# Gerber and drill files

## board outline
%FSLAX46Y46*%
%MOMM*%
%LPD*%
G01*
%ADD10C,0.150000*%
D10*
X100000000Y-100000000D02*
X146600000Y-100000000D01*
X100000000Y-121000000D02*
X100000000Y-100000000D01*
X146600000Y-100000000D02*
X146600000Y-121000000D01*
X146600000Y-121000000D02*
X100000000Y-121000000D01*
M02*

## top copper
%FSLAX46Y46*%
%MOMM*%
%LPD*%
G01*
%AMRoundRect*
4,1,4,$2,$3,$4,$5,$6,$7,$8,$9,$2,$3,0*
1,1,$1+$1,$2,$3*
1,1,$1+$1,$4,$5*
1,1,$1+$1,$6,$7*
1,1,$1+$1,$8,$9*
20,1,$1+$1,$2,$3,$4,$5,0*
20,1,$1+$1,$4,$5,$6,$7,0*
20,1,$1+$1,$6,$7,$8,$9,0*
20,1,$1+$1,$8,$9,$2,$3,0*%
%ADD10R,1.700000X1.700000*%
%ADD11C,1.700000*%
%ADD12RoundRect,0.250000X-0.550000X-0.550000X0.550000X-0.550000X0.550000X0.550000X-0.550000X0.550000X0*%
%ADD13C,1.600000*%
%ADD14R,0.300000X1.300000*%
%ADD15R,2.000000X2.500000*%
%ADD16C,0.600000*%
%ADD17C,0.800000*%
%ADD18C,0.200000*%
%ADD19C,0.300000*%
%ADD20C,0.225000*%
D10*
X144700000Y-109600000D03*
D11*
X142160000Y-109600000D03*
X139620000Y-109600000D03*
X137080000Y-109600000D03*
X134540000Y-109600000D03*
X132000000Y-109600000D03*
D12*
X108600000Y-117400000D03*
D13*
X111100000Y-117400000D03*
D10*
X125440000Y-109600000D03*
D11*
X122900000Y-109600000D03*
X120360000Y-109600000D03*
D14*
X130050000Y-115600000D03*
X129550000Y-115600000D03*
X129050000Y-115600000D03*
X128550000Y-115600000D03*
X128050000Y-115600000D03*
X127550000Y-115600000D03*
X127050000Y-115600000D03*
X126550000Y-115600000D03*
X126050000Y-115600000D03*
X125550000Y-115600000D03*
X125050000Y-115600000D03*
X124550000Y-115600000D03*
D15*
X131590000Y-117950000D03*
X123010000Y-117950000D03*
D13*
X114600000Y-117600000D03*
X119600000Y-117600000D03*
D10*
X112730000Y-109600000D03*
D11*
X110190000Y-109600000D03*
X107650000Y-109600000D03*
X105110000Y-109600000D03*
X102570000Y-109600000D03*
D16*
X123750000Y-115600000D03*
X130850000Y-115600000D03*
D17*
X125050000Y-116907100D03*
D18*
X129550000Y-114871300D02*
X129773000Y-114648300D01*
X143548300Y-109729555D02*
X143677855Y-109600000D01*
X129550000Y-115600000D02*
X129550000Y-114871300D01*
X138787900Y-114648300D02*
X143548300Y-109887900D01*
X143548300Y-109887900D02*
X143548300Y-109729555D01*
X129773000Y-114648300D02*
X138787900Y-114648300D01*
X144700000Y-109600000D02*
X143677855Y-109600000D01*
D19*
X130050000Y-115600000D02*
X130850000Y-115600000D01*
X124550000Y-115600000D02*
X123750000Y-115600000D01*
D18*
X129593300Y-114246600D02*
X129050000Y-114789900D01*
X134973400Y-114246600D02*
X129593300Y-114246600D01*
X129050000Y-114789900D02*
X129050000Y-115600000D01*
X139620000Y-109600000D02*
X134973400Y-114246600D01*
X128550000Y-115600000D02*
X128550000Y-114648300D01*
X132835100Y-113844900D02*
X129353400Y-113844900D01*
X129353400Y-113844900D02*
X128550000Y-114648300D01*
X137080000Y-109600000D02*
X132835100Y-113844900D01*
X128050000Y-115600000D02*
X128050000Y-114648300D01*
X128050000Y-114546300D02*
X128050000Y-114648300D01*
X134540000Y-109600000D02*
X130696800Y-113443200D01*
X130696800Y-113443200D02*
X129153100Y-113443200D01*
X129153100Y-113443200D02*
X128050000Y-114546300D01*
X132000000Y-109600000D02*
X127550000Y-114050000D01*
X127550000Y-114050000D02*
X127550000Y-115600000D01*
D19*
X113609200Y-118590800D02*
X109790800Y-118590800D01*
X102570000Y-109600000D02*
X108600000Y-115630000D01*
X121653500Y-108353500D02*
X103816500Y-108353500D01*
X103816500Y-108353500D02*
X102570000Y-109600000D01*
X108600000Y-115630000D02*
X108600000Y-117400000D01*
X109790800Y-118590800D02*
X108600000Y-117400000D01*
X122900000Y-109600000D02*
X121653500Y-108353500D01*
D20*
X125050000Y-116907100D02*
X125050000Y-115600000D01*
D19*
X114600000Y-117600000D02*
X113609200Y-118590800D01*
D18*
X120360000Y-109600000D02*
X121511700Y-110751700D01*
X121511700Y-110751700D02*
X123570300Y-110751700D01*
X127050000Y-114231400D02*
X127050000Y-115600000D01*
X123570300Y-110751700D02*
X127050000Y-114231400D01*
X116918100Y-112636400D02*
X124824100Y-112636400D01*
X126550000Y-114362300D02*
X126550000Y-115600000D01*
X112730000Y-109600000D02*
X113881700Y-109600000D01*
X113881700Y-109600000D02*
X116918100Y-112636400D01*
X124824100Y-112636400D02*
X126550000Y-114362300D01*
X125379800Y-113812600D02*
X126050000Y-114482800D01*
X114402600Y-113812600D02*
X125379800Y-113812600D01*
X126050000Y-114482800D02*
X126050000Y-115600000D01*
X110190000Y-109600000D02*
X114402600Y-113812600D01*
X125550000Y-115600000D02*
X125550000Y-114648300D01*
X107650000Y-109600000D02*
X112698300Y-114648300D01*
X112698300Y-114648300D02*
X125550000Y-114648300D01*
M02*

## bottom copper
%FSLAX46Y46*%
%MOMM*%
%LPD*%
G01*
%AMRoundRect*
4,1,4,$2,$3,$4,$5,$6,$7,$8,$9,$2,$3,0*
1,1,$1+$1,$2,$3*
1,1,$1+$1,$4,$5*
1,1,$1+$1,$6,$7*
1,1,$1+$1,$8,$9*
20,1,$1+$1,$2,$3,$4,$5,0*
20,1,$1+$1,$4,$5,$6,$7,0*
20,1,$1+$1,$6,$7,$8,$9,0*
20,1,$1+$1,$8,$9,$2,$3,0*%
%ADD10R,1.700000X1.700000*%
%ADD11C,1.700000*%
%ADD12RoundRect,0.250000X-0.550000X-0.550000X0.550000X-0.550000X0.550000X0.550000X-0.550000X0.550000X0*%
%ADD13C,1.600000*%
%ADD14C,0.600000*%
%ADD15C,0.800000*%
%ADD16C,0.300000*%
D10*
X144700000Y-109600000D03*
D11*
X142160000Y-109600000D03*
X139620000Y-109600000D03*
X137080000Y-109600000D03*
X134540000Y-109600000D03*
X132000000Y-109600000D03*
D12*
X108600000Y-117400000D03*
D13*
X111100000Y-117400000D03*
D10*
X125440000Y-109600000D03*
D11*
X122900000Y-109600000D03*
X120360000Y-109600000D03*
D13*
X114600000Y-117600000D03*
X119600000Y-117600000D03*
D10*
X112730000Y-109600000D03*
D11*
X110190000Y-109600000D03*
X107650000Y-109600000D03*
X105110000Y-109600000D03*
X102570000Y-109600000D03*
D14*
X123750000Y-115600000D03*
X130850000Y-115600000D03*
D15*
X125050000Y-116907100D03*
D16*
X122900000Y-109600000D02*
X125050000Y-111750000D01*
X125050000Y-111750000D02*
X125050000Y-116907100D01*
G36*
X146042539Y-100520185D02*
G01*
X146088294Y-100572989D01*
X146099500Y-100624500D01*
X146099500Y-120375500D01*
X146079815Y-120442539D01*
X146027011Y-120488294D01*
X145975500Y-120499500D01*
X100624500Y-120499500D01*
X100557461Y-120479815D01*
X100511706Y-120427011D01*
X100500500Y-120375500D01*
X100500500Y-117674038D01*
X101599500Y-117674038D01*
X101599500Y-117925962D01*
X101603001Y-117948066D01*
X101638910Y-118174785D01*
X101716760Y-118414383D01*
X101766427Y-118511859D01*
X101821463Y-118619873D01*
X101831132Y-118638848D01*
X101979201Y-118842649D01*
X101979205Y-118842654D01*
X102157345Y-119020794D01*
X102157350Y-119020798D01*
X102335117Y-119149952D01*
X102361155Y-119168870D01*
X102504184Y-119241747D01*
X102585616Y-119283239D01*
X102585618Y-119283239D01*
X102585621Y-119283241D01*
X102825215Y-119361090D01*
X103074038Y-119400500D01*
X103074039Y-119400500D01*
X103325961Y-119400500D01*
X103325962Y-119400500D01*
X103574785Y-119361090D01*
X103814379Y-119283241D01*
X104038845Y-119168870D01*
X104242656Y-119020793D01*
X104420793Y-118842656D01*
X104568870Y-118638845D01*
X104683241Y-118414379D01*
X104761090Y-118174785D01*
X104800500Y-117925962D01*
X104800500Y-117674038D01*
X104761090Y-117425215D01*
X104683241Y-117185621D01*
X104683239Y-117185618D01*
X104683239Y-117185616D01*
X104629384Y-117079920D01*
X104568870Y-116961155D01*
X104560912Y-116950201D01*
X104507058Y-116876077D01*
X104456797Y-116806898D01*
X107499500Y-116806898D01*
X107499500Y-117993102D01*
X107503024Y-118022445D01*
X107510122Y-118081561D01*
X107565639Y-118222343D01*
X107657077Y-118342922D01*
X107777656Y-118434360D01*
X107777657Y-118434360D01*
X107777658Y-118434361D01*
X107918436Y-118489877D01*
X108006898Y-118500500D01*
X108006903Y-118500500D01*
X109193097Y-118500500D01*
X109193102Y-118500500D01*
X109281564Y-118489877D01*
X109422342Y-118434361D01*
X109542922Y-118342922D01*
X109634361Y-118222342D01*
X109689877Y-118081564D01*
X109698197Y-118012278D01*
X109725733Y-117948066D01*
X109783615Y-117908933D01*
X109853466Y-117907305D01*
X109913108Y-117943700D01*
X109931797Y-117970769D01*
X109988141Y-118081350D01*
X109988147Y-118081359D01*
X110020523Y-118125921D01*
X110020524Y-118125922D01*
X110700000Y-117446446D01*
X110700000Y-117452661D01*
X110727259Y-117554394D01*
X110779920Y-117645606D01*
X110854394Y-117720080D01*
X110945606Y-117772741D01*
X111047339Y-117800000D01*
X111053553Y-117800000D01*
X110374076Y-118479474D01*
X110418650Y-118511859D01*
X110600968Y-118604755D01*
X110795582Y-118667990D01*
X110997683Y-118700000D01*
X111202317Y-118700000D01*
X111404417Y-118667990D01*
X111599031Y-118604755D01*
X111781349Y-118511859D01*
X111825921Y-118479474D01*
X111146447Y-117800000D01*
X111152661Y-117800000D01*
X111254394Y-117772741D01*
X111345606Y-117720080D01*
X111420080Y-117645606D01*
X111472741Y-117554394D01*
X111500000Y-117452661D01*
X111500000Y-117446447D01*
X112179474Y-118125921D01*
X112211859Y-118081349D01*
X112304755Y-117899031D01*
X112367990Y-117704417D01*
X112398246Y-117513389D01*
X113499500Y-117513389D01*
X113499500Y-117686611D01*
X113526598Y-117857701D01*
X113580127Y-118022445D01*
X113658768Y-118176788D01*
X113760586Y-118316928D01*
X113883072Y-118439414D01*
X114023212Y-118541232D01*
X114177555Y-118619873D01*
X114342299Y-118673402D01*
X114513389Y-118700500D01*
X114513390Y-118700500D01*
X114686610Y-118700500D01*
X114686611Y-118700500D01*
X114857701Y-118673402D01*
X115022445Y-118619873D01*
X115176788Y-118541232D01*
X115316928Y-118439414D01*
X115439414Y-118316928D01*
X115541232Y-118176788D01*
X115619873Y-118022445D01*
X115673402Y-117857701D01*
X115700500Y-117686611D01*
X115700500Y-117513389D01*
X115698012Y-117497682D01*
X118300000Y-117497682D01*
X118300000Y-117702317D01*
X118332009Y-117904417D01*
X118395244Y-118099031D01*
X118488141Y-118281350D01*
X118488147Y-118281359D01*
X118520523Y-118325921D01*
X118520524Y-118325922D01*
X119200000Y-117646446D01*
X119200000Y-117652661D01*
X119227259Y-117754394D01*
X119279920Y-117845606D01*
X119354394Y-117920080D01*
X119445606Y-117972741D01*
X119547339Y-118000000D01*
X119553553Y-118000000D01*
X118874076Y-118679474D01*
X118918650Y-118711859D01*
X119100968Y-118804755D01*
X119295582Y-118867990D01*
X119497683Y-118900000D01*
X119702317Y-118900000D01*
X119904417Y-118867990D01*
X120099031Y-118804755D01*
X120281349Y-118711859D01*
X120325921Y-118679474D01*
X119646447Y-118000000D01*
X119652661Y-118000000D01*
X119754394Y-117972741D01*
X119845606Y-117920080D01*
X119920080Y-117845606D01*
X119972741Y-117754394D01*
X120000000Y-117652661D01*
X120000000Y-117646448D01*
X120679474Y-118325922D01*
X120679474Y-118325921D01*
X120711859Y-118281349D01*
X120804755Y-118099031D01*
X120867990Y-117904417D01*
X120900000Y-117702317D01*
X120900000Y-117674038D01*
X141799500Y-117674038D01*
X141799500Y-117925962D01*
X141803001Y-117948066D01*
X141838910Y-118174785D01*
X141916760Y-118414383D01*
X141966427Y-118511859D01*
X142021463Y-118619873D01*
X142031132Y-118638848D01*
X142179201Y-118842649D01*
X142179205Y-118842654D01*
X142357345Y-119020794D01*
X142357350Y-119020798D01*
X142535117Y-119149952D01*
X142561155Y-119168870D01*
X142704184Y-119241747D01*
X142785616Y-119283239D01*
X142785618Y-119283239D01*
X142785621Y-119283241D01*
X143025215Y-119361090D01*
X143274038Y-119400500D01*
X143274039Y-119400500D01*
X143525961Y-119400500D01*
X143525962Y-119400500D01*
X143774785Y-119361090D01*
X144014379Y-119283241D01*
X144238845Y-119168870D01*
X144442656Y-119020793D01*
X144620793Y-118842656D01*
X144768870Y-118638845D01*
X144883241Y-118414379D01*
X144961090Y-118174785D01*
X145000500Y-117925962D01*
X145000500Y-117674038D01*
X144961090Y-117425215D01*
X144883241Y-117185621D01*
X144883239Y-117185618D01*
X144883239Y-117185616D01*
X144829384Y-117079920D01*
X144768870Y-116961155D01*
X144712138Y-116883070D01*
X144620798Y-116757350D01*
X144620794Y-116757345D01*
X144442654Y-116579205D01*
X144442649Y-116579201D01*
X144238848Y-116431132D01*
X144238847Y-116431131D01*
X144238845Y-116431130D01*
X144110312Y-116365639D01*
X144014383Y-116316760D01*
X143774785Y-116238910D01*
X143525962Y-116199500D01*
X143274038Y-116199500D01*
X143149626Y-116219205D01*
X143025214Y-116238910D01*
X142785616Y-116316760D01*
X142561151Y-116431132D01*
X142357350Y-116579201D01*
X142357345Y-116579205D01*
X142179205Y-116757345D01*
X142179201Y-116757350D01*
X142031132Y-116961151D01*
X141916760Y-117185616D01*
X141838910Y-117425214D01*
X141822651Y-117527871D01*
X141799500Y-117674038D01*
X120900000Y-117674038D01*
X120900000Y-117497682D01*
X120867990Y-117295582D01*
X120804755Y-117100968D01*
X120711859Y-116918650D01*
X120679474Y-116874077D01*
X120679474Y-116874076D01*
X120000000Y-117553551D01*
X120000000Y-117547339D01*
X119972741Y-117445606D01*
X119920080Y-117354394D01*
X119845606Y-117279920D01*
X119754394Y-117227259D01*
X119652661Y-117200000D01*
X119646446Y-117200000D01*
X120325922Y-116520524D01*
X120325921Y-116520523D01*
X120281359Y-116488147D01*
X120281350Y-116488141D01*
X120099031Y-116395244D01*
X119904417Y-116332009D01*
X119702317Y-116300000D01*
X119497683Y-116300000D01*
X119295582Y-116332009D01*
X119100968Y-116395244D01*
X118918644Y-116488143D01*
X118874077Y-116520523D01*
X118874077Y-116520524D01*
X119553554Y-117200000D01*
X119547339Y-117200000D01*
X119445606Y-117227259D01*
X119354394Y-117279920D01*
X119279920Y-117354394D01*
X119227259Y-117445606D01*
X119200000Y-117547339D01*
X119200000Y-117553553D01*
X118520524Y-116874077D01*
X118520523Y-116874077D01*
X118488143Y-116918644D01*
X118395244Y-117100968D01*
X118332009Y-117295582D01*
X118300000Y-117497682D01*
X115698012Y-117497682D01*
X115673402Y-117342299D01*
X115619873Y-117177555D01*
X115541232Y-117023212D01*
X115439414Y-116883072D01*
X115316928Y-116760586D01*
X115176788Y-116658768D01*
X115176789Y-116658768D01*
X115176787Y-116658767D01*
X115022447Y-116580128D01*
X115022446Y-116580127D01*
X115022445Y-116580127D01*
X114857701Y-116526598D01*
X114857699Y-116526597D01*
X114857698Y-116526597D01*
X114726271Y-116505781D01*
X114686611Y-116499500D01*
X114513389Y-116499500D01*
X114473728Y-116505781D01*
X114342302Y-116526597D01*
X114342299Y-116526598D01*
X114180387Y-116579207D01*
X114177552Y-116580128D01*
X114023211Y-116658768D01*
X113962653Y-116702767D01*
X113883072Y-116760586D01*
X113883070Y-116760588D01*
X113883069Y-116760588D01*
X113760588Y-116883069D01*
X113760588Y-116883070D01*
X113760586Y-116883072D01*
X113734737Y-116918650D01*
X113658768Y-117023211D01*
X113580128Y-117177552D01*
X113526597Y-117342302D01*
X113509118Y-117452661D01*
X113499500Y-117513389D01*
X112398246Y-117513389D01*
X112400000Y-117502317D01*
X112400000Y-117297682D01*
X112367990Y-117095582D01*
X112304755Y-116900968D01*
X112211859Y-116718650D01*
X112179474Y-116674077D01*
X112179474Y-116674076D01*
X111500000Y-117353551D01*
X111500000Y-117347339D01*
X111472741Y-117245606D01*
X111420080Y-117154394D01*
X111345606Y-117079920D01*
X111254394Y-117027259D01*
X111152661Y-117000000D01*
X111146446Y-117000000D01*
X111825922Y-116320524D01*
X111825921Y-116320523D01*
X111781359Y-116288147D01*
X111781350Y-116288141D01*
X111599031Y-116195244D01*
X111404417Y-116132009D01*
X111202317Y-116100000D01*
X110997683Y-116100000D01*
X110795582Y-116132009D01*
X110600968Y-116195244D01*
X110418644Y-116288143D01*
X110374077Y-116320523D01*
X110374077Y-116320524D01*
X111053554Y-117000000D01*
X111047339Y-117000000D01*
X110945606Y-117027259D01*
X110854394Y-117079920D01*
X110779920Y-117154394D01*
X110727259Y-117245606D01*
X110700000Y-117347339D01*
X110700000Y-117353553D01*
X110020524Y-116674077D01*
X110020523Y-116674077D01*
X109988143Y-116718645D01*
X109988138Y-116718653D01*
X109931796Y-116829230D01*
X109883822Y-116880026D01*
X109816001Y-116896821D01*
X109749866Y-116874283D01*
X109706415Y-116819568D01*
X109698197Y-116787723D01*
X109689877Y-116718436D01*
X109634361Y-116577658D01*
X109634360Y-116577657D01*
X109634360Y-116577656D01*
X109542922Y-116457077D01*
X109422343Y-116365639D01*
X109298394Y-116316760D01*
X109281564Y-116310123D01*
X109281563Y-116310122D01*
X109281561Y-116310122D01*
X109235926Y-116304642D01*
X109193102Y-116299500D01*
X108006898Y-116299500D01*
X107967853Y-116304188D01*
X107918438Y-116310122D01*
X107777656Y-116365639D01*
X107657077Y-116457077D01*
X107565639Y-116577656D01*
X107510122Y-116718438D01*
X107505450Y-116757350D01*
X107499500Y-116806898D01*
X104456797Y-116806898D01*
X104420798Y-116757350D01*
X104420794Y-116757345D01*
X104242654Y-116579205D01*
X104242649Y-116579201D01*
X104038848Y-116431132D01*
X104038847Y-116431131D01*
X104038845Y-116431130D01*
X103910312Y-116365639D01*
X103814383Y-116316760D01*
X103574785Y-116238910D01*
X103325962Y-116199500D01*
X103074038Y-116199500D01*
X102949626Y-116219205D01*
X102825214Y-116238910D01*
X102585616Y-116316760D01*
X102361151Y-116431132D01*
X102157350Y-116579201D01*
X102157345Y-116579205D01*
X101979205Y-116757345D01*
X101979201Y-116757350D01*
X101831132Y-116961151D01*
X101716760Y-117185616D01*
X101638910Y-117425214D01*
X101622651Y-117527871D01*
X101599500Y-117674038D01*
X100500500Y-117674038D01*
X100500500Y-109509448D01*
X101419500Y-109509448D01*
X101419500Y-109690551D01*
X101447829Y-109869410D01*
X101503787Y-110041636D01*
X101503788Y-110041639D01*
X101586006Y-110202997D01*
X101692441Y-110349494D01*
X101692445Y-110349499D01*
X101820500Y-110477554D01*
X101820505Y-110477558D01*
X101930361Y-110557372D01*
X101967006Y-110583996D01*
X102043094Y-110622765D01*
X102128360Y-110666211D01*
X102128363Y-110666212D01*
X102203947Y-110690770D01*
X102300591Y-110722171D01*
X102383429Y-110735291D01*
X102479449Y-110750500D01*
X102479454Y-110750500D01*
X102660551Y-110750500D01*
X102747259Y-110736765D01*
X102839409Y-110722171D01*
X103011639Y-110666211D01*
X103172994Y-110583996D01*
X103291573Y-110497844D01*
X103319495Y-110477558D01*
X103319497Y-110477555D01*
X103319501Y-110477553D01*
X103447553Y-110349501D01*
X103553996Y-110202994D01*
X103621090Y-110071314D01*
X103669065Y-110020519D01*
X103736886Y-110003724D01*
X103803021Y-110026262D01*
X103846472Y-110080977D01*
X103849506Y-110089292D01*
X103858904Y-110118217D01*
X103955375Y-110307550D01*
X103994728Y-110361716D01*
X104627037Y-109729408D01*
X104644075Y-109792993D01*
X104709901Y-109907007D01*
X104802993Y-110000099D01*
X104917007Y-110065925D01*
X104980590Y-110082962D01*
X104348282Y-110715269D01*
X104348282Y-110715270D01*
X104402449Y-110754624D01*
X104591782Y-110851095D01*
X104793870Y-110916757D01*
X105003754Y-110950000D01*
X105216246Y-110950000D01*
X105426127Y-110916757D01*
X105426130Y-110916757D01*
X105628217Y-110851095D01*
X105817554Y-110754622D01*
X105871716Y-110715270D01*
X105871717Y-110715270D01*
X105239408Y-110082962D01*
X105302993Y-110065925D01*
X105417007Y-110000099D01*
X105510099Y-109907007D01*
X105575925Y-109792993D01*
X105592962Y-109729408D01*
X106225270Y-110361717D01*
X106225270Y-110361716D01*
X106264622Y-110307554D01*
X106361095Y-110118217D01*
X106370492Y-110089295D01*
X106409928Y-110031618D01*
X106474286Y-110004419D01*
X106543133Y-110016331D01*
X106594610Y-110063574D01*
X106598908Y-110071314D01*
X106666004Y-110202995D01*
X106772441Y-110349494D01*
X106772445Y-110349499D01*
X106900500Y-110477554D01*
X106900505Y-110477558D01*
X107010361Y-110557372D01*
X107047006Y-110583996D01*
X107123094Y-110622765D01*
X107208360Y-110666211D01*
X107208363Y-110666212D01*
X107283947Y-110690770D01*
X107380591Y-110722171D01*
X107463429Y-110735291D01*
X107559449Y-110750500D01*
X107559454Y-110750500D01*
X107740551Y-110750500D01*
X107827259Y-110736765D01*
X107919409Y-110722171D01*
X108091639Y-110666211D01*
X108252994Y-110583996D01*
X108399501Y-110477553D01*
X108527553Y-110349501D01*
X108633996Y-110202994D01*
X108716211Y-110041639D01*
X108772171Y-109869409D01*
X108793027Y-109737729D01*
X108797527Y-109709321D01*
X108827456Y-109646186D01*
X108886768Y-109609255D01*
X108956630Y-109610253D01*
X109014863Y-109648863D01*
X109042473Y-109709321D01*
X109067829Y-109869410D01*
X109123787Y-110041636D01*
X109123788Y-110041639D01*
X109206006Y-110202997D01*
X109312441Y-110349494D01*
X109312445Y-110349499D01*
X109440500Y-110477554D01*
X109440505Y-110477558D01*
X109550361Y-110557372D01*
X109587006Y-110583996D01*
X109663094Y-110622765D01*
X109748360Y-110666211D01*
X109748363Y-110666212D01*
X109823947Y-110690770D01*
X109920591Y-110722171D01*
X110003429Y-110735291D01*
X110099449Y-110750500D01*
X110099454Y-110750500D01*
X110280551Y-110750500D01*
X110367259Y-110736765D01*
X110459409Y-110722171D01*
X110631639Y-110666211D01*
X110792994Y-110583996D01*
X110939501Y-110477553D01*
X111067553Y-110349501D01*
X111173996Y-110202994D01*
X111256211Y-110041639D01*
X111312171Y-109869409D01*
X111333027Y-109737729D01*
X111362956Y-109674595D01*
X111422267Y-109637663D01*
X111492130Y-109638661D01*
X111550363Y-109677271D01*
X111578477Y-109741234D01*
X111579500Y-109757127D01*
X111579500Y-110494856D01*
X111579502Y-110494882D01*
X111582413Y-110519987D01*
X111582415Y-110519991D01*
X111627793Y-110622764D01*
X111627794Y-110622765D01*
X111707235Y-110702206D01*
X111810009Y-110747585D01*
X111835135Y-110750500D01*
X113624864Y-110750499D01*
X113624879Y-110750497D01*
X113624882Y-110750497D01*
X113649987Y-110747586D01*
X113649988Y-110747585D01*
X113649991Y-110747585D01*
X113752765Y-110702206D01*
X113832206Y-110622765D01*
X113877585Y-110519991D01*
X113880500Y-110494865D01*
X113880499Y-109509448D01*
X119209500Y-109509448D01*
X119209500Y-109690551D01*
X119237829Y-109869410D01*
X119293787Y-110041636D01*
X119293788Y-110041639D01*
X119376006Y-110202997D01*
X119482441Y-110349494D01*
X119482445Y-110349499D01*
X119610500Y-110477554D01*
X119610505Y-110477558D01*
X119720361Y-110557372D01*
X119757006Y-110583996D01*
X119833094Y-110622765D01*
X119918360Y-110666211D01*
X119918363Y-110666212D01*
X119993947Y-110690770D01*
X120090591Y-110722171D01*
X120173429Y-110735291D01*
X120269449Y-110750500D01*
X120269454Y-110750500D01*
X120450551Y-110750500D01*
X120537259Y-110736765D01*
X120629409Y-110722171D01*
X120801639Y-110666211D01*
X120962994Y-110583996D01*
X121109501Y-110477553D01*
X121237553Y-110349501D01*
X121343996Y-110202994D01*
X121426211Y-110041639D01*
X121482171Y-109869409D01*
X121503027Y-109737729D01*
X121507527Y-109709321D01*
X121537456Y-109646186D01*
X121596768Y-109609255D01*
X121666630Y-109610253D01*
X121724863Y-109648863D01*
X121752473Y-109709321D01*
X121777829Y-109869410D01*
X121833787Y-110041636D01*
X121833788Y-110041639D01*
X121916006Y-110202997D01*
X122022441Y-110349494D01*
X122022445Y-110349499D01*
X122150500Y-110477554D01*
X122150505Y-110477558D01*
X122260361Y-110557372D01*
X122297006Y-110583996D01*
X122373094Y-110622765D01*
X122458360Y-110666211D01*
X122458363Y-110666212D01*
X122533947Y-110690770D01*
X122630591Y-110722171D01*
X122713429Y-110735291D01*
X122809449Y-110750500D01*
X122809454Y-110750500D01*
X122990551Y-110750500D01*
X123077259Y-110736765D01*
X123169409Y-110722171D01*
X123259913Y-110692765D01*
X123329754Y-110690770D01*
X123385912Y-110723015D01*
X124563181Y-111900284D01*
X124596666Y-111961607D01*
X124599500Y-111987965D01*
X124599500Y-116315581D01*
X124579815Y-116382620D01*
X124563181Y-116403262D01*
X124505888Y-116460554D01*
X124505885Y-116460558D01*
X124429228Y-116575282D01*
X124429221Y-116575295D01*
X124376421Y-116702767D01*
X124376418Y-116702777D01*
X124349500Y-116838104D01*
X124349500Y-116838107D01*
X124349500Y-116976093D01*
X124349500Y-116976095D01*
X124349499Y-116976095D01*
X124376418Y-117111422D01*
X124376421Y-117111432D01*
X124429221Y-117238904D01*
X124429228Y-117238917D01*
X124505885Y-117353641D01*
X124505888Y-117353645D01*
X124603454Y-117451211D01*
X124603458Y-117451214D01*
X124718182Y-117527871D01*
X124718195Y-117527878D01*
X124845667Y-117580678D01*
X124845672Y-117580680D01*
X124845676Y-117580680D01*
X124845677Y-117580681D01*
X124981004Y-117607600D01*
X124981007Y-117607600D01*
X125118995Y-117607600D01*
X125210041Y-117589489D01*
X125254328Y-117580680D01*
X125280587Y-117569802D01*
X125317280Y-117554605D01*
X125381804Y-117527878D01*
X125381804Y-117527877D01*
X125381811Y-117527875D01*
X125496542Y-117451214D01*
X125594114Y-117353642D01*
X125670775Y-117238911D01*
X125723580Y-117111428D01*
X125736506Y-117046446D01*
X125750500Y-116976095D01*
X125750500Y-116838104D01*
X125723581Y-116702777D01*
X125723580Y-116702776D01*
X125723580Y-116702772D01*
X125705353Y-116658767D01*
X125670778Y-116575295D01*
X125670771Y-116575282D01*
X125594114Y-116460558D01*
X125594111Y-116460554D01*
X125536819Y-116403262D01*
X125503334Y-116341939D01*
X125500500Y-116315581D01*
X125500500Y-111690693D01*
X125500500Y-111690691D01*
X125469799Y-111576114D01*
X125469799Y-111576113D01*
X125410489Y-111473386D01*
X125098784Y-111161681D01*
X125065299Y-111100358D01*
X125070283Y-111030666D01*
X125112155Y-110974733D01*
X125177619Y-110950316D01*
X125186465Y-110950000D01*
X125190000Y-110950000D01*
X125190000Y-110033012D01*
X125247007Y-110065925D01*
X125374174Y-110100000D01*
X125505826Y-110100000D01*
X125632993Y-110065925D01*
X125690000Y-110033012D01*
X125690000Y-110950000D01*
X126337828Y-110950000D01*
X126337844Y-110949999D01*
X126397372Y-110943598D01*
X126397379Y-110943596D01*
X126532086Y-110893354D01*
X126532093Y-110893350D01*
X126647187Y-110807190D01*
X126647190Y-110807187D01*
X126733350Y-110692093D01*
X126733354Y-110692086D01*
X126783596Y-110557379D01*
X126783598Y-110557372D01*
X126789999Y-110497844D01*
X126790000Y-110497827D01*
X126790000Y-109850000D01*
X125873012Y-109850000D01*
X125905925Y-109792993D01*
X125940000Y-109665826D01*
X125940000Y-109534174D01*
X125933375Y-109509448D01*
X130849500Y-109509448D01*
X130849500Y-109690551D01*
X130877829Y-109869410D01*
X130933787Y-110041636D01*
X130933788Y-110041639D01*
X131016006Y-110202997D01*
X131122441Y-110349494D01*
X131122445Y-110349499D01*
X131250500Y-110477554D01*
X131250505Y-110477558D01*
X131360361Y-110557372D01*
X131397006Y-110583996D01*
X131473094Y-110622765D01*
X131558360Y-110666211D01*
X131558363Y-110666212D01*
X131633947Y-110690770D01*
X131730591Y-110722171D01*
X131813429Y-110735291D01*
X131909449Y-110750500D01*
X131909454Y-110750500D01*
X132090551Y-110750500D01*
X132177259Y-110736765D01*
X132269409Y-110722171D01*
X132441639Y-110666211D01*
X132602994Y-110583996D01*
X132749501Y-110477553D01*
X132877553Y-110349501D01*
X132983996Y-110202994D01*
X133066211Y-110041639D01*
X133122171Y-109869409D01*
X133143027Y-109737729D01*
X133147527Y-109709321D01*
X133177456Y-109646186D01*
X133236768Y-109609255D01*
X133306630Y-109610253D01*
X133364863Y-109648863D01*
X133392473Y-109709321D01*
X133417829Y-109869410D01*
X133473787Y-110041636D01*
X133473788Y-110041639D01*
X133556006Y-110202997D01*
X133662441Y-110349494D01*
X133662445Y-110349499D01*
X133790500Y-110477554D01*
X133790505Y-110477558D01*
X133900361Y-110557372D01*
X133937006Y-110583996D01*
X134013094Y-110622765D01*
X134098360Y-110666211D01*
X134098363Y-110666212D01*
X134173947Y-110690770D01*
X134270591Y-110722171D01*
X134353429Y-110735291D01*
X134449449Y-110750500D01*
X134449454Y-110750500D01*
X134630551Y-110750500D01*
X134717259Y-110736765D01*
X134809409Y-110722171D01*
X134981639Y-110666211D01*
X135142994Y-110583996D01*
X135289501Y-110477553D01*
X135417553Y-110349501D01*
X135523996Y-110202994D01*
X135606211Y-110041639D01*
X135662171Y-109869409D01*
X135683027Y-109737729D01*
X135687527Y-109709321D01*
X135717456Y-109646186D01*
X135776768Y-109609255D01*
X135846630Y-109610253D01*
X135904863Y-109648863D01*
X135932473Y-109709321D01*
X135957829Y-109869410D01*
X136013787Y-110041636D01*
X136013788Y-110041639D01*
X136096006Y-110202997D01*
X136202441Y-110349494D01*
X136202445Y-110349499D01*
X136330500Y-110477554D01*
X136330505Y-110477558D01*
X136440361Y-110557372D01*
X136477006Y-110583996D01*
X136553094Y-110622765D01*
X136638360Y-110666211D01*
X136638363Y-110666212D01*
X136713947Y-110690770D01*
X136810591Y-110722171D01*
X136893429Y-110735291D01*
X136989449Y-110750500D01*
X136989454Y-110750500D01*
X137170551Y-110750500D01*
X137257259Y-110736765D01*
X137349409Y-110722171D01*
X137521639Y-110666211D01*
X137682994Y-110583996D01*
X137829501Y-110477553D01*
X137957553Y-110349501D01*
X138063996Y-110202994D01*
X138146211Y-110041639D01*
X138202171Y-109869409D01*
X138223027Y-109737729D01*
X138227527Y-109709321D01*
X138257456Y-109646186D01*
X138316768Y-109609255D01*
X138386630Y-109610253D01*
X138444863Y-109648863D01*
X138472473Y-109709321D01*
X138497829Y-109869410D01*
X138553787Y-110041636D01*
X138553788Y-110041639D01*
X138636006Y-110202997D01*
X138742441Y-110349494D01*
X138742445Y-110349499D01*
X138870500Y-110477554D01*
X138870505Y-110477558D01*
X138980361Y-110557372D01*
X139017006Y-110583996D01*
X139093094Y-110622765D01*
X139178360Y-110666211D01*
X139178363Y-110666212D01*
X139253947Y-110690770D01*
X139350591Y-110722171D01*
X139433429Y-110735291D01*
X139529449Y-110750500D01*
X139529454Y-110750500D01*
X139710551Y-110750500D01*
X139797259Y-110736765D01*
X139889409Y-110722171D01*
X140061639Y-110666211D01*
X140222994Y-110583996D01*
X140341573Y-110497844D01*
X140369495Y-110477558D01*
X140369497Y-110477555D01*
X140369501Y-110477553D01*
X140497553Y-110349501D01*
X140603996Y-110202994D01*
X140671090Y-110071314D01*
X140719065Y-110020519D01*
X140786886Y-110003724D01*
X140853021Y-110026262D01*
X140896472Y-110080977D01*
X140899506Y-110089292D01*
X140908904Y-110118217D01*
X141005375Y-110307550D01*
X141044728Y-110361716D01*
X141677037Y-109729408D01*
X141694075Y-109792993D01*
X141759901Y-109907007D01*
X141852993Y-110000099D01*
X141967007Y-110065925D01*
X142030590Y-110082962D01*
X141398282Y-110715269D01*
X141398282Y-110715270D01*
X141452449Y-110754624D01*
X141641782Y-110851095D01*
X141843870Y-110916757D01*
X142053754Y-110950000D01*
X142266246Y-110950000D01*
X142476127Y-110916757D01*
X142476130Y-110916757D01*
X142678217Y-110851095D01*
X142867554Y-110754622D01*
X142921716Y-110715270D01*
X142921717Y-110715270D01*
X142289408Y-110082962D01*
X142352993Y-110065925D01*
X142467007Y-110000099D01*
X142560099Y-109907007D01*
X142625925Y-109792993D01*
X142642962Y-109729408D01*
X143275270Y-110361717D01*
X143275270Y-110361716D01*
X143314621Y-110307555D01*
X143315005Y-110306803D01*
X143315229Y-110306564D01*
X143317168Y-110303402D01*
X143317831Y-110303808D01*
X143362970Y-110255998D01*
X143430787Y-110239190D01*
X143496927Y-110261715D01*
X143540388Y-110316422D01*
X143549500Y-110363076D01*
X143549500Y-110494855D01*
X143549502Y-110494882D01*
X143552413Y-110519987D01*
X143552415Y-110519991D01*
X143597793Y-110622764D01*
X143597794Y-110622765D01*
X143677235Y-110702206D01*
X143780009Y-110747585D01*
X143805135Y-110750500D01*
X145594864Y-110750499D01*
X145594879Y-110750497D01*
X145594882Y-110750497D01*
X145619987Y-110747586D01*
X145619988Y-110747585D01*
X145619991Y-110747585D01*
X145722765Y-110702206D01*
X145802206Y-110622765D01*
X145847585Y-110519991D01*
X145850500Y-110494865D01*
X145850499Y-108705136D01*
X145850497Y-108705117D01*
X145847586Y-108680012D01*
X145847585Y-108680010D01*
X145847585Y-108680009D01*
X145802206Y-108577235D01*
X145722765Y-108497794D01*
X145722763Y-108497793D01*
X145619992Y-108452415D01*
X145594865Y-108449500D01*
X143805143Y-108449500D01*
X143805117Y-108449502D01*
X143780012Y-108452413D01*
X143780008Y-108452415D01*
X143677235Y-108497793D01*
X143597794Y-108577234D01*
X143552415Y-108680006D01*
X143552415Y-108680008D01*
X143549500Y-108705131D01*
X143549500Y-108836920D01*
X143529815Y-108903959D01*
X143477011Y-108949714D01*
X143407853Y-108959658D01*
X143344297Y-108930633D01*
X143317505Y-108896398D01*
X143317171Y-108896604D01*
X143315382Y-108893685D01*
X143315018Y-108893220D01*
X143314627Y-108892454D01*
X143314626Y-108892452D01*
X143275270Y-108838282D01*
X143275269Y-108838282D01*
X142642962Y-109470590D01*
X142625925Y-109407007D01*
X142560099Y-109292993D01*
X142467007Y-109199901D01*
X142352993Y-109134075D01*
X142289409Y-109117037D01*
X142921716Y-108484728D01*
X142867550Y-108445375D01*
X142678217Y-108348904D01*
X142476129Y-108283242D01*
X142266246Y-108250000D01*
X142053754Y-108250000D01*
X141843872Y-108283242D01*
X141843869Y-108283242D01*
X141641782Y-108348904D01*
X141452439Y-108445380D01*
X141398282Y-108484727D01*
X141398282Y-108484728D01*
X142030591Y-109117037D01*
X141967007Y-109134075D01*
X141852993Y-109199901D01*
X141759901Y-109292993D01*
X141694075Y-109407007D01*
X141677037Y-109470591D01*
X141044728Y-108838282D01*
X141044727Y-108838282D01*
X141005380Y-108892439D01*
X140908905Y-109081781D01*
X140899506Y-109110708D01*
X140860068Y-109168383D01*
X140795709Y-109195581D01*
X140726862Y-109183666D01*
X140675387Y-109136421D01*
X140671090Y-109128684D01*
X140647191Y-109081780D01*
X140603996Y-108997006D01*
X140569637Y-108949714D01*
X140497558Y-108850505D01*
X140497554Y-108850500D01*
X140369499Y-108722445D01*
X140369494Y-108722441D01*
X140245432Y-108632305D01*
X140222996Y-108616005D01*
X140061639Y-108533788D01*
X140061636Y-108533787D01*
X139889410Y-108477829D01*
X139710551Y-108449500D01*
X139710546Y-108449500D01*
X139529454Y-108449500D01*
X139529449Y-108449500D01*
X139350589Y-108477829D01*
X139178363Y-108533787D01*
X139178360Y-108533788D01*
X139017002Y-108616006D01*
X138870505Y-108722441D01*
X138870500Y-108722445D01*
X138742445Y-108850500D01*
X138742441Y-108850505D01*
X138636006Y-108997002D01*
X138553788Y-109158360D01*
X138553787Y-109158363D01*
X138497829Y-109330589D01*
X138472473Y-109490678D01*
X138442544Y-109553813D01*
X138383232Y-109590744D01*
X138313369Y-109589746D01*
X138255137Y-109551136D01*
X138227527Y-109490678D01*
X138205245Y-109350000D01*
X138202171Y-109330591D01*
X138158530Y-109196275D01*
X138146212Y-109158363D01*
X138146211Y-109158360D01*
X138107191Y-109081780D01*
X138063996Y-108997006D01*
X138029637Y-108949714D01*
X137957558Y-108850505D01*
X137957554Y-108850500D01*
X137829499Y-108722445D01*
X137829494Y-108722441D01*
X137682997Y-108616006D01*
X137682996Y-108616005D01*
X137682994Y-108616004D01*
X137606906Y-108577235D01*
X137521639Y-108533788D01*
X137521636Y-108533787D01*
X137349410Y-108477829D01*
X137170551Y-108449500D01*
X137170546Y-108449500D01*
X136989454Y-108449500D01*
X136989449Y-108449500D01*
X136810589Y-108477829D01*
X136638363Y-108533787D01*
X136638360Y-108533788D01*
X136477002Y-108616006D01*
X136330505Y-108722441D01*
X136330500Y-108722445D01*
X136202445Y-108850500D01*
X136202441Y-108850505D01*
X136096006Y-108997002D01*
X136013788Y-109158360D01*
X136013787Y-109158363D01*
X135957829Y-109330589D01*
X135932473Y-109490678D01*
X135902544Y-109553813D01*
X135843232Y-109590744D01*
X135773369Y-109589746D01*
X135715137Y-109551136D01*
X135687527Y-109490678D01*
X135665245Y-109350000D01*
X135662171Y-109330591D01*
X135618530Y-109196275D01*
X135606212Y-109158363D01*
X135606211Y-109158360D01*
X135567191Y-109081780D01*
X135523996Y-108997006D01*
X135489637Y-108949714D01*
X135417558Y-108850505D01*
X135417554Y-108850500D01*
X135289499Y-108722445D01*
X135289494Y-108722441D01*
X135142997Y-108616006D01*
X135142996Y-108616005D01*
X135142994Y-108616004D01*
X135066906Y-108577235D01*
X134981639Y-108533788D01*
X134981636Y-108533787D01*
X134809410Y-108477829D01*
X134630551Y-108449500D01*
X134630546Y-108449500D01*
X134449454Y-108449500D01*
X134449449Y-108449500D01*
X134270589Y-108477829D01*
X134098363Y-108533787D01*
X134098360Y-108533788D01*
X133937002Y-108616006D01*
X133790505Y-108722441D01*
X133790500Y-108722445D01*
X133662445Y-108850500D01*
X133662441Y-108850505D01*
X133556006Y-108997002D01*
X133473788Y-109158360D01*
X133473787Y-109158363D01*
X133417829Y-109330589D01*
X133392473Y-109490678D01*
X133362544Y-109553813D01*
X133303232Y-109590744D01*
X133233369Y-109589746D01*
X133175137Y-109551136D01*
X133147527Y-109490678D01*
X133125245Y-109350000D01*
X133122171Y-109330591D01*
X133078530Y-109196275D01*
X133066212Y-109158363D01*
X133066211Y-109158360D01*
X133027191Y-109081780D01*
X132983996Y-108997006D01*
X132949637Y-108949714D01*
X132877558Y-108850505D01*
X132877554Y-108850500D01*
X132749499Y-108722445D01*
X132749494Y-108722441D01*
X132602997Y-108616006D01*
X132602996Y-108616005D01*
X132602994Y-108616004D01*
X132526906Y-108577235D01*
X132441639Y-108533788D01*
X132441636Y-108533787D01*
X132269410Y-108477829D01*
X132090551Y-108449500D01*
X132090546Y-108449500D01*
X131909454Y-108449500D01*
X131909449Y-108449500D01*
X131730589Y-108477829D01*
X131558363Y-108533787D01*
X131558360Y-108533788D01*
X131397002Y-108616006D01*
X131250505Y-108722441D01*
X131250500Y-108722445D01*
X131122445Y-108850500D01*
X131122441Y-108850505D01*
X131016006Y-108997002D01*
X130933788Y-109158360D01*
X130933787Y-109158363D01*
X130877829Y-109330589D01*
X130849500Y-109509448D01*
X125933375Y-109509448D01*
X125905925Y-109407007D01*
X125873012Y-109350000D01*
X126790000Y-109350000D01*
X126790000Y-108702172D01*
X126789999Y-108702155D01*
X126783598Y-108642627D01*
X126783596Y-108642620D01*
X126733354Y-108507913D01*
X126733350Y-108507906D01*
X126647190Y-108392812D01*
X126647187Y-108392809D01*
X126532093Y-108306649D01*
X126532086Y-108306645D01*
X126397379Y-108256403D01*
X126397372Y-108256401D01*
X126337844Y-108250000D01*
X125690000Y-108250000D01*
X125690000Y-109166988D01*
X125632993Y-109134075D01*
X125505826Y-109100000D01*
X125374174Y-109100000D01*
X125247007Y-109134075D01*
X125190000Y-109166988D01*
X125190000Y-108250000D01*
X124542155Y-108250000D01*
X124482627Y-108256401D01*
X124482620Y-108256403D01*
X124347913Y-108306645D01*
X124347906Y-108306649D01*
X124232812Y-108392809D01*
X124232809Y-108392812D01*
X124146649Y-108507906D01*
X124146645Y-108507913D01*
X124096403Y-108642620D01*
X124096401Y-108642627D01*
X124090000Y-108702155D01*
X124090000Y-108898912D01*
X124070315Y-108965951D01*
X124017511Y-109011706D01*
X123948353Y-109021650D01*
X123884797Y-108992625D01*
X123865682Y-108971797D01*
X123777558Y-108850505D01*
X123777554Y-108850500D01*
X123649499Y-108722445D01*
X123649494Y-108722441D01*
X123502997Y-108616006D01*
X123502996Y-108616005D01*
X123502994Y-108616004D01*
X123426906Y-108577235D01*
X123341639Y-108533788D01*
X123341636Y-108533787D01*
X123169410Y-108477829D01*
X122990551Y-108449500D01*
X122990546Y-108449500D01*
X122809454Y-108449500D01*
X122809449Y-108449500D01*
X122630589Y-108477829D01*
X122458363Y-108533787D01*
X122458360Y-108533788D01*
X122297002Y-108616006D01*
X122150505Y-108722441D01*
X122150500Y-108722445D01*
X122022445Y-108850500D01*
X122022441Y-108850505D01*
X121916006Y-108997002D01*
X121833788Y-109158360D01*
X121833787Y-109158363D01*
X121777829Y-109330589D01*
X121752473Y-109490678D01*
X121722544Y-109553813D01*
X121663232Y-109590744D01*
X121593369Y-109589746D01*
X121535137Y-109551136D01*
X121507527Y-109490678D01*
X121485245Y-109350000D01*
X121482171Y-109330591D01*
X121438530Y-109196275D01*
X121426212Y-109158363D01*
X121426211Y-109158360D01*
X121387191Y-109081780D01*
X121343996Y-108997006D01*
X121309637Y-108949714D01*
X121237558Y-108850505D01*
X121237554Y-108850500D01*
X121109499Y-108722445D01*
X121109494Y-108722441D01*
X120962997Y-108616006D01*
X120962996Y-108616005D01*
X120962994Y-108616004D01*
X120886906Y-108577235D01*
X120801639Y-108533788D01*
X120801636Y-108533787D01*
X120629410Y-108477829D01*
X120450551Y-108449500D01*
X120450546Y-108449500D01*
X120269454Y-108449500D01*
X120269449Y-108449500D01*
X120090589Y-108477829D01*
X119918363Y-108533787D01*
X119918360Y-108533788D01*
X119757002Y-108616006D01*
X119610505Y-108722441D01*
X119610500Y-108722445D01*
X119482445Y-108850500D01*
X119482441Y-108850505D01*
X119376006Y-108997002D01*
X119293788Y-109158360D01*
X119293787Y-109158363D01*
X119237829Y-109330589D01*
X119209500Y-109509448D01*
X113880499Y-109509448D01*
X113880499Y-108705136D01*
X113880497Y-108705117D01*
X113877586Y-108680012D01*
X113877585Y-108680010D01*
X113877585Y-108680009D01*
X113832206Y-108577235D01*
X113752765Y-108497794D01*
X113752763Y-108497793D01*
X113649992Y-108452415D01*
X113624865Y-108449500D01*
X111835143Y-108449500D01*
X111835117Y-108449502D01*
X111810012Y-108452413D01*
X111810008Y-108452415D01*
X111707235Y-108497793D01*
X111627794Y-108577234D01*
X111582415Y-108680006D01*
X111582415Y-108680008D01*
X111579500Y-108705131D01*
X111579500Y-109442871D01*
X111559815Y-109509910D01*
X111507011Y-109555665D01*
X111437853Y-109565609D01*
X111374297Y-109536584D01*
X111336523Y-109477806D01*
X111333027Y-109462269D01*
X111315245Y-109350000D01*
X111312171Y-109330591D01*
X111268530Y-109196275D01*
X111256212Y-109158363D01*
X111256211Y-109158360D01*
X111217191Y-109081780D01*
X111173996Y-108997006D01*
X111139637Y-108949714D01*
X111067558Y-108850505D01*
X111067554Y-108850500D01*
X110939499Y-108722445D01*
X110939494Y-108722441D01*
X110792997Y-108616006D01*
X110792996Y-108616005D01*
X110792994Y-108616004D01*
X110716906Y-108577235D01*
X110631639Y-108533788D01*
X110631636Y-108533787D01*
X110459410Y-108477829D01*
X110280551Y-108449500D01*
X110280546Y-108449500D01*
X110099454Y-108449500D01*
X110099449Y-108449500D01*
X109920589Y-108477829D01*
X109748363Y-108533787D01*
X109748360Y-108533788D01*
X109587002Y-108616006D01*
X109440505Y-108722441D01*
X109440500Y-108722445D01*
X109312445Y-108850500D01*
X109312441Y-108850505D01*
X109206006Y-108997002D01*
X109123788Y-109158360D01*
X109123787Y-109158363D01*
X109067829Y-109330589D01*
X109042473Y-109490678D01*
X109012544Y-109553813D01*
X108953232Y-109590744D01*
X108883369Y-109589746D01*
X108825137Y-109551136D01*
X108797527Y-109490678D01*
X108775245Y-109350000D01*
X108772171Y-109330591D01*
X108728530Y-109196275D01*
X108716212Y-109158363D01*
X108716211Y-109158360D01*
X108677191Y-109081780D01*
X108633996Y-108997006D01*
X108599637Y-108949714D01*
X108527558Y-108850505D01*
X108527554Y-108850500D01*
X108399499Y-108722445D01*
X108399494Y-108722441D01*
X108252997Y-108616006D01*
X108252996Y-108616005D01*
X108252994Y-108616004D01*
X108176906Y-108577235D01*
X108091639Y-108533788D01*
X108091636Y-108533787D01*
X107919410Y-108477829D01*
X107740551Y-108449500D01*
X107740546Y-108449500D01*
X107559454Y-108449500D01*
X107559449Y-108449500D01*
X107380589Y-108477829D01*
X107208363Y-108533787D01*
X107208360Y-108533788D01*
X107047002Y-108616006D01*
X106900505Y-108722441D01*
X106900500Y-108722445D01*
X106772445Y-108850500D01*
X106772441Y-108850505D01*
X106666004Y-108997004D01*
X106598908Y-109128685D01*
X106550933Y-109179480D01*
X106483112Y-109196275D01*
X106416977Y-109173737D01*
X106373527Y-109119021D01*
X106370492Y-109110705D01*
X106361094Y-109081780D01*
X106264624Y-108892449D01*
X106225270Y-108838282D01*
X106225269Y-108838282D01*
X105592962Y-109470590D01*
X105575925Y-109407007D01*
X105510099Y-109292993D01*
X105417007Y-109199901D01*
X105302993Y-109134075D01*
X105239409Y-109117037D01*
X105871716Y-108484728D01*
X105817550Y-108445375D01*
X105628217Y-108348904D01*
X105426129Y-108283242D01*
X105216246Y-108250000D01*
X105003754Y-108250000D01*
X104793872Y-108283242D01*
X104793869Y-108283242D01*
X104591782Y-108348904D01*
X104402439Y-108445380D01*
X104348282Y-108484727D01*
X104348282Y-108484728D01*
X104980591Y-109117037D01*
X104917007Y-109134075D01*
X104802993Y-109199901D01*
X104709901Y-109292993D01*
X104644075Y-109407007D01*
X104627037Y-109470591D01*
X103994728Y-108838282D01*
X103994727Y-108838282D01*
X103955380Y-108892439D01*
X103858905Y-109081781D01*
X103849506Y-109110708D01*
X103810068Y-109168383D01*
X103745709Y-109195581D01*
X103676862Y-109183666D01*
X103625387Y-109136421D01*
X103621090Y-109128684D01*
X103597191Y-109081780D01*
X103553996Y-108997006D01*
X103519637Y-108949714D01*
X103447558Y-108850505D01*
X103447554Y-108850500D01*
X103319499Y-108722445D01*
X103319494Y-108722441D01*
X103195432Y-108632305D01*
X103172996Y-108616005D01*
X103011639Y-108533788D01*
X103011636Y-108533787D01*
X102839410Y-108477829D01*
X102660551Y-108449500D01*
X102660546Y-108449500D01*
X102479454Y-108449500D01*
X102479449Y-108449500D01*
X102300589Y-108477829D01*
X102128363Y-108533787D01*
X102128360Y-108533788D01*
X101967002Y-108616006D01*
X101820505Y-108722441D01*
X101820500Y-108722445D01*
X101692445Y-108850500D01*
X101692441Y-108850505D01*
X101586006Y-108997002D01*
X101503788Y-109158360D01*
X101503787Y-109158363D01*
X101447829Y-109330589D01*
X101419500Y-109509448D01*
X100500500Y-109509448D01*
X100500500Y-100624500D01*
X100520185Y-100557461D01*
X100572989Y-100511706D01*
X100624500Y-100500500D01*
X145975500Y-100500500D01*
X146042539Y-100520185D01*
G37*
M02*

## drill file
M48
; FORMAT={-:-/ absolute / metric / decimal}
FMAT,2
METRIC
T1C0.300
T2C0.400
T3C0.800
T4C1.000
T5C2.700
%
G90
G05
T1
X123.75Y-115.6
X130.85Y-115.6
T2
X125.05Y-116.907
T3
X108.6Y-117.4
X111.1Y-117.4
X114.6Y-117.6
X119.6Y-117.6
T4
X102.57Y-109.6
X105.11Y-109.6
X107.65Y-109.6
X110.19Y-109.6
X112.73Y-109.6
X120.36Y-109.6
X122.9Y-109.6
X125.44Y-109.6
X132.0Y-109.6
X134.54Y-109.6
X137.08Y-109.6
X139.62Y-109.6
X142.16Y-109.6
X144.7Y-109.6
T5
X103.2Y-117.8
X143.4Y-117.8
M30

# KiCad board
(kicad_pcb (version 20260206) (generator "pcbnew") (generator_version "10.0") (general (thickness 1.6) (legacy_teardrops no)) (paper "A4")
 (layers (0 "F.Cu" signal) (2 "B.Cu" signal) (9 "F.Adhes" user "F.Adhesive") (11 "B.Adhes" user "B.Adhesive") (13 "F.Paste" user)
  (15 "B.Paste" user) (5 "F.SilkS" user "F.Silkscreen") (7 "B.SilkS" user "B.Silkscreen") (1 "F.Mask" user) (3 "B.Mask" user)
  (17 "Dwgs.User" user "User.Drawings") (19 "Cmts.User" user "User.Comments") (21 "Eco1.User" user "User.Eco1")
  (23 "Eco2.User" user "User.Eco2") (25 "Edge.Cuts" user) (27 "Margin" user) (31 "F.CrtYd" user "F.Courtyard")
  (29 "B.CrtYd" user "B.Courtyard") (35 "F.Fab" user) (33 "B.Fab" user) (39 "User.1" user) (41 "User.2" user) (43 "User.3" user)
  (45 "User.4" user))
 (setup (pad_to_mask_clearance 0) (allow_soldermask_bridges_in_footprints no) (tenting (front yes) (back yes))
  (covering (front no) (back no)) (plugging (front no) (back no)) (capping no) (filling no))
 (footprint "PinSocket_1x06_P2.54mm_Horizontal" (layer "F.Cu") (at 144.7 109.6 -90)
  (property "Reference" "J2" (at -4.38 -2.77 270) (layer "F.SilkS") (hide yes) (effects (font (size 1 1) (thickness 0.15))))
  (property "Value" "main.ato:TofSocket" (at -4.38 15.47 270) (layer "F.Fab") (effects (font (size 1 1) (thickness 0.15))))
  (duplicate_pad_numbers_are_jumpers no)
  (pad "1" thru_hole rect (at 0 0 270) (size 1.7 1.7) (drill 1) (layers "*.Cu" "*.Mask") (remove_unused_layers no) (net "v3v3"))
  (pad "2" thru_hole circle (at 0 2.54 270) (size 1.7 1.7) (drill 1) (layers "*.Cu" "*.Mask") (remove_unused_layers no) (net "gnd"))
  (pad "3" thru_hole circle (at 0 5.08 270) (size 1.7 1.7) (drill 1) (layers "*.Cu" "*.Mask") (remove_unused_layers no) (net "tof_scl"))
  (pad "4" thru_hole circle (at 0 7.62 270) (size 1.7 1.7) (drill 1) (layers "*.Cu" "*.Mask") (remove_unused_layers no) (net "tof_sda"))
  (pad "5" thru_hole circle (at 0 10.16 270) (size 1.7 1.7) (drill 1) (layers "*.Cu" "*.Mask") (remove_unused_layers no) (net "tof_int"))
  (pad "6" thru_hole circle (at 0 12.7 270) (size 1.7 1.7) (drill 1) (layers "*.Cu" "*.Mask") (remove_unused_layers no) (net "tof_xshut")))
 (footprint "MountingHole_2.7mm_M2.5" (layer "F.Cu") (at 143.4 117.8)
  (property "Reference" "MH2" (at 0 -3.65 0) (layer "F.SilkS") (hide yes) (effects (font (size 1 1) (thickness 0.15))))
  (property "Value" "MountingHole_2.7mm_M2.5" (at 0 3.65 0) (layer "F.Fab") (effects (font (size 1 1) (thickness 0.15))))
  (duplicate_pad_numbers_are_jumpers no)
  (pad "" np_thru_hole circle (at 0 0) (size 2.7 2.7) (drill 2.7) (layers "*.Cu" "*.Mask")))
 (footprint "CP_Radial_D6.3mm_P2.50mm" (layer "F.Cu") (at 108.6 117.4)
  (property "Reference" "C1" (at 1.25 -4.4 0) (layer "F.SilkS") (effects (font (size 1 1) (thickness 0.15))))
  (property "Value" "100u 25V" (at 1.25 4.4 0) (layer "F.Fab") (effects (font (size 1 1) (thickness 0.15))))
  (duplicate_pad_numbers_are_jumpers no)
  (pad "1" thru_hole roundrect (at 0 0) (size 1.6 1.6) (drill 0.8) (layers "*.Cu" "*.Mask") (remove_unused_layers no)
   (roundrect_rratio 0.15625) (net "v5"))
  (pad "2" thru_hole circle (at 2.5 0) (size 1.6 1.6) (drill 0.8) (layers "*.Cu" "*.Mask") (remove_unused_layers no) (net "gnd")))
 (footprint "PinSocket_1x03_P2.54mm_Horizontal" (layer "F.Cu") (at 125.44 109.6 -90)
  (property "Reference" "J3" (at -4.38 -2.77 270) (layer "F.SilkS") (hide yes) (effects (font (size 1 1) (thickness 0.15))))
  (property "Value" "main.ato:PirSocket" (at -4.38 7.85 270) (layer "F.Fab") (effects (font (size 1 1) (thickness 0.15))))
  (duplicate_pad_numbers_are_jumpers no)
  (pad "1" thru_hole rect (at 0 0 270) (size 1.7 1.7) (drill 1) (layers "*.Cu" "*.Mask") (remove_unused_layers no) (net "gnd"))
  (pad "2" thru_hole circle (at 0 2.54 270) (size 1.7 1.7) (drill 1) (layers "*.Cu" "*.Mask") (remove_unused_layers no) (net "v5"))
  (pad "3" thru_hole circle (at 0 5.08 270) (size 1.7 1.7) (drill 1) (layers "*.Cu" "*.Mask") (remove_unused_layers no) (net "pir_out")))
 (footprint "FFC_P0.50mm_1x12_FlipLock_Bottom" (layer "F.Cu") (at 127.3 115.6 180)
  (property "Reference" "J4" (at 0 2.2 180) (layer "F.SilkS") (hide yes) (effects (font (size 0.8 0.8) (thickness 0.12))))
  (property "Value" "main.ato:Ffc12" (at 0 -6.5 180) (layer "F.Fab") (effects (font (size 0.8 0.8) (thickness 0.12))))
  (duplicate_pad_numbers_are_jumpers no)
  (pad "1" smd rect (at -2.75 0 180) (size 0.3 1.3) (layers "F.Cu" "F.Mask" "F.Paste") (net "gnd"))
  (pad "2" smd rect (at -2.25 0 180) (size 0.3 1.3) (layers "F.Cu" "F.Mask" "F.Paste") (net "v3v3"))
  (pad "3" smd rect (at -1.75 0 180) (size 0.3 1.3) (layers "F.Cu" "F.Mask" "F.Paste") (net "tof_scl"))
  (pad "4" smd rect (at -1.25 0 180) (size 0.3 1.3) (layers "F.Cu" "F.Mask" "F.Paste") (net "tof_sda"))
  (pad "5" smd rect (at -0.75 0 180) (size 0.3 1.3) (layers "F.Cu" "F.Mask" "F.Paste") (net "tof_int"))
  (pad "6" smd rect (at -0.25 0 180) (size 0.3 1.3) (layers "F.Cu" "F.Mask" "F.Paste") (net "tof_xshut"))
  (pad "7" smd rect (at 0.25 0 180) (size 0.3 1.3) (layers "F.Cu" "F.Mask" "F.Paste") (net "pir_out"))
  (pad "8" smd rect (at 0.75 0 180) (size 0.3 1.3) (layers "F.Cu" "F.Mask" "F.Paste") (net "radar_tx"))
  (pad "9" smd rect (at 1.25 0 180) (size 0.3 1.3) (layers "F.Cu" "F.Mask" "F.Paste") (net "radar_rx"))
  (pad "10" smd rect (at 1.75 0 180) (size 0.3 1.3) (layers "F.Cu" "F.Mask" "F.Paste") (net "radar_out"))
  (pad "11" smd rect (at 2.25 0 180) (size 0.3 1.3) (layers "F.Cu" "F.Mask" "F.Paste") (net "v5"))
  (pad "12" smd rect (at 2.75 0 180) (size 0.3 1.3) (layers "F.Cu" "F.Mask" "F.Paste") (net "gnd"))
  (pad "MP" smd rect (at -4.29 -2.35 180) (size 2 2.5) (layers "F.Cu" "F.Mask" "F.Paste"))
  (pad "MP" smd rect (at 4.29 -2.35 180) (size 2 2.5) (layers "F.Cu" "F.Mask" "F.Paste")))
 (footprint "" (layer "F.Cu") (at 100 100)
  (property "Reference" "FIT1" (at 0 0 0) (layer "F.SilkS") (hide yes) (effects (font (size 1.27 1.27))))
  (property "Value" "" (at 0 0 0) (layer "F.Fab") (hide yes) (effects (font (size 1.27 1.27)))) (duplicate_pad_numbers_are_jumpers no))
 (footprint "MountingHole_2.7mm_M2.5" (layer "F.Cu") (at 103.2 117.8)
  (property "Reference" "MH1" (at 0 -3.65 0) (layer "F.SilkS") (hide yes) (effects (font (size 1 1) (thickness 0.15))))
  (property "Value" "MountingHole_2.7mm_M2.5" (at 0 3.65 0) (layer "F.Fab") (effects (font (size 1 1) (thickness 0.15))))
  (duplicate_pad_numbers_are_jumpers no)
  (pad "" np_thru_hole circle (at 0 0) (size 2.7 2.7) (drill 2.7) (layers "*.Cu" "*.Mask")))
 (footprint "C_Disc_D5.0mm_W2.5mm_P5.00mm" (layer "F.Cu") (at 114.6 117.6)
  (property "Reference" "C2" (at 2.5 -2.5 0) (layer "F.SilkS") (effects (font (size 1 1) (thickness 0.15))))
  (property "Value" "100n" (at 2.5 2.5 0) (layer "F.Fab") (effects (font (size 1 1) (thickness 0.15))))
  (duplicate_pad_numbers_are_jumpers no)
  (pad "1" thru_hole circle (at 0 0) (size 1.6 1.6) (drill 0.8) (layers "*.Cu" "*.Mask") (remove_unused_layers no) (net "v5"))
  (pad "2" thru_hole circle (at 5 0) (size 1.6 1.6) (drill 0.8) (layers "*.Cu" "*.Mask") (remove_unused_layers no) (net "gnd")))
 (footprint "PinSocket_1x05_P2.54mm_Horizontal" (layer "F.Cu") (at 112.73 109.6 -90)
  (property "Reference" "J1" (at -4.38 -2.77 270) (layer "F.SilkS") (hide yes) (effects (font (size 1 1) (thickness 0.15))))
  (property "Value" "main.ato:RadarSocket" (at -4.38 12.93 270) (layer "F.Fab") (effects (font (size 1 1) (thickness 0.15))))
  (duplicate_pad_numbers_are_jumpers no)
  (pad "1" thru_hole rect (at 0 0 270) (size 1.7 1.7) (drill 1) (layers "*.Cu" "*.Mask") (remove_unused_layers no) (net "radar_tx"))
  (pad "2" thru_hole circle (at 0 2.54 270) (size 1.7 1.7) (drill 1) (layers "*.Cu" "*.Mask") (remove_unused_layers no) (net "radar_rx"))
  (pad "3" thru_hole circle (at 0 5.08 270) (size 1.7 1.7) (drill 1) (layers "*.Cu" "*.Mask") (remove_unused_layers no) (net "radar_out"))
  (pad "4" thru_hole circle (at 0 7.62 270) (size 1.7 1.7) (drill 1) (layers "*.Cu" "*.Mask") (remove_unused_layers no) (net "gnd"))
  (pad "5" thru_hole circle (at 0 10.16 270) (size 1.7 1.7) (drill 1) (layers "*.Cu" "*.Mask") (remove_unused_layers no) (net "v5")))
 (gr_line (start 100 100) (end 146.6 100) (stroke (width 0.15) (type default)) (layer "Edge.Cuts"))
 (gr_line (start 100 121) (end 100 100) (stroke (width 0.15) (type default)) (layer "Edge.Cuts"))
 (gr_line (start 146.6 100) (end 146.6 121) (stroke (width 0.15) (type default)) (layer "Edge.Cuts"))
 (gr_line (start 146.6 121) (end 100 121) (stroke (width 0.15) (type default)) (layer "Edge.Cuts"))
 (segment (start 129.55 114.8713) (end 129.773 114.6483) (width 0.2) (locked yes) (layer "F.Cu") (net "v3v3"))
 (segment (start 143.5483 109.729555) (end 143.677855 109.6) (width 0.2) (locked yes) (layer "F.Cu") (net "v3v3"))
 (segment (start 129.55 115.6) (end 129.55 114.8713) (width 0.2) (locked yes) (layer "F.Cu") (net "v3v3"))
 (segment (start 138.7879 114.6483) (end 143.5483 109.8879) (width 0.2) (locked yes) (layer "F.Cu") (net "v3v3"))
 (segment (start 143.5483 109.8879) (end 143.5483 109.729555) (width 0.2) (locked yes) (layer "F.Cu") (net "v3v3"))
 (segment (start 129.773 114.6483) (end 138.7879 114.6483) (width 0.2) (locked yes) (layer "F.Cu") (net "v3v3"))
 (segment (start 144.7 109.6) (end 143.677855 109.6) (width 0.2) (locked yes) (layer "F.Cu") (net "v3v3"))
 (segment (start 130.05 115.6) (end 130.85 115.6) (width 0.3) (locked yes) (layer "F.Cu") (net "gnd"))
 (segment (start 124.55 115.6) (end 123.75 115.6) (width 0.3) (locked yes) (layer "F.Cu") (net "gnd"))
 (via (at 123.75 115.6) (size 0.6) (drill 0.3) (layers "F.Cu" "B.Cu") (locked yes) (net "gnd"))
 (via (at 130.85 115.6) (size 0.6) (drill 0.3) (layers "F.Cu" "B.Cu") (locked yes) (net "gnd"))
 (segment (start 129.5933 114.2466) (end 129.05 114.7899) (width 0.2) (locked yes) (layer "F.Cu") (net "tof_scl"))
 (segment (start 134.9734 114.2466) (end 129.5933 114.2466) (width 0.2) (locked yes) (layer "F.Cu") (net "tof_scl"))
 (segment (start 129.05 114.7899) (end 129.05 115.6) (width 0.2) (locked yes) (layer "F.Cu") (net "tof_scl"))
 (segment (start 139.62 109.6) (end 134.9734 114.2466) (width 0.2) (locked yes) (layer "F.Cu") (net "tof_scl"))
 (segment (start 128.55 115.6) (end 128.55 114.6483) (width 0.2) (locked yes) (layer "F.Cu") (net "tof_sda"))
 (segment (start 132.8351 113.8449) (end 129.3534 113.8449) (width 0.2) (locked yes) (layer "F.Cu") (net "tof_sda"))
 (segment (start 129.3534 113.8449) (end 128.55 114.6483) (width 0.2) (locked yes) (layer "F.Cu") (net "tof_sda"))
 (segment (start 137.08 109.6) (end 132.8351 113.8449) (width 0.2) (locked yes) (layer "F.Cu") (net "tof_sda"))
 (segment (start 128.05 115.6) (end 128.05 114.6483) (width 0.2) (locked yes) (layer "F.Cu") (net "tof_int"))
 (segment (start 128.05 114.5463) (end 128.05 114.6483) (width 0.2) (locked yes) (layer "F.Cu") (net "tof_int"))
 (segment (start 134.54 109.6) (end 130.6968 113.4432) (width 0.2) (locked yes) (layer "F.Cu") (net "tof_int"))
 (segment (start 130.6968 113.4432) (end 129.1531 113.4432) (width 0.2) (locked yes) (layer "F.Cu") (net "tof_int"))
 (segment (start 129.1531 113.4432) (end 128.05 114.5463) (width 0.2) (locked yes) (layer "F.Cu") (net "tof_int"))
 (segment (start 132 109.6) (end 127.55 114.05) (width 0.2) (locked yes) (layer "F.Cu") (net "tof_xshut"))
 (segment (start 127.55 114.05) (end 127.55 115.6) (width 0.2) (locked yes) (layer "F.Cu") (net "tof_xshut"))
 (segment (start 113.6092 118.5908) (end 109.7908 118.5908) (width 0.3) (locked yes) (layer "F.Cu") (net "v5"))
 (segment (start 102.57 109.6) (end 108.6 115.63) (width 0.3) (locked yes) (layer "F.Cu") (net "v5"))
 (segment (start 121.6535 108.3535) (end 103.8165 108.3535) (width 0.3) (locked yes) (layer "F.Cu") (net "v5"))
 (segment (start 103.8165 108.3535) (end 102.57 109.6) (width 0.3) (locked yes) (layer "F.Cu") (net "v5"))
 (segment (start 108.6 115.63) (end 108.6 117.4) (width 0.3) (locked yes) (layer "F.Cu") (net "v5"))
 (segment (start 109.7908 118.5908) (end 108.6 117.4) (width 0.3) (locked yes) (layer "F.Cu") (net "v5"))
 (segment (start 122.9 109.6) (end 121.6535 108.3535) (width 0.3) (locked yes) (layer "F.Cu") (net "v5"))
 (segment (start 125.05 116.9071) (end 125.05 115.6) (width 0.225) (layer "F.Cu") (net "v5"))
 (segment (start 114.6 117.6) (end 113.6092 118.5908) (width 0.3) (locked yes) (layer "F.Cu") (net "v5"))
 (via (at 125.05 116.9071) (size 0.8) (drill 0.4) (layers "F.Cu" "B.Cu") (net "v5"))
 (segment (start 122.9 109.6) (end 125.05 111.75) (width 0.3) (layer "B.Cu") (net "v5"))
 (segment (start 125.05 111.75) (end 125.05 116.9071) (width 0.3) (layer "B.Cu") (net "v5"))
 (segment (start 120.36 109.6) (end 121.5117 110.7517) (width 0.2) (locked yes) (layer "F.Cu") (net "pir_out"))
 (segment (start 121.5117 110.7517) (end 123.5703 110.7517) (width 0.2) (locked yes) (layer "F.Cu") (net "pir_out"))
 (segment (start 127.05 114.2314) (end 127.05 115.6) (width 0.2) (locked yes) (layer "F.Cu") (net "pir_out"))
 (segment (start 123.5703 110.7517) (end 127.05 114.2314) (width 0.2) (locked yes) (layer "F.Cu") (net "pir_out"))
 (segment (start 116.9181 112.6364) (end 124.8241 112.6364) (width 0.2) (locked yes) (layer "F.Cu") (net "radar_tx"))
 (segment (start 126.55 114.3623) (end 126.55 115.6) (width 0.2) (locked yes) (layer "F.Cu") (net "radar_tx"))
 (segment (start 112.73 109.6) (end 113.8817 109.6) (width 0.2) (locked yes) (layer "F.Cu") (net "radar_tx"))
 (segment (start 113.8817 109.6) (end 116.9181 112.6364) (width 0.2) (locked yes) (layer "F.Cu") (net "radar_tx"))
 (segment (start 124.8241 112.6364) (end 126.55 114.3623) (width 0.2) (locked yes) (layer "F.Cu") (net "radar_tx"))
 (segment (start 125.3798 113.8126) (end 126.05 114.4828) (width 0.2) (locked yes) (layer "F.Cu") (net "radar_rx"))
 (segment (start 114.4026 113.8126) (end 125.3798 113.8126) (width 0.2) (locked yes) (layer "F.Cu") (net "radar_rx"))
 (segment (start 126.05 114.4828) (end 126.05 115.6) (width 0.2) (locked yes) (layer "F.Cu") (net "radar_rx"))
 (segment (start 110.19 109.6) (end 114.4026 113.8126) (width 0.2) (locked yes) (layer "F.Cu") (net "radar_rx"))
 (segment (start 125.55 115.6) (end 125.55 114.6483) (width 0.2) (locked yes) (layer "F.Cu") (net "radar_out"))
 (segment (start 107.65 109.6) (end 112.6983 114.6483) (width 0.2) (locked yes) (layer "F.Cu") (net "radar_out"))
 (segment (start 112.6983 114.6483) (end 125.55 114.6483) (width 0.2) (locked yes) (layer "F.Cu") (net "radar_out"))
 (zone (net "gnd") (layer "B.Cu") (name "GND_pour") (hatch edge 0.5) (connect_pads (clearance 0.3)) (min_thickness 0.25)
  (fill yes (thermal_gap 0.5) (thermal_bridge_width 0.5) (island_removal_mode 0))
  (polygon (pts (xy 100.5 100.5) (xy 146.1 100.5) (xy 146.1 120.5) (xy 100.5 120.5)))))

